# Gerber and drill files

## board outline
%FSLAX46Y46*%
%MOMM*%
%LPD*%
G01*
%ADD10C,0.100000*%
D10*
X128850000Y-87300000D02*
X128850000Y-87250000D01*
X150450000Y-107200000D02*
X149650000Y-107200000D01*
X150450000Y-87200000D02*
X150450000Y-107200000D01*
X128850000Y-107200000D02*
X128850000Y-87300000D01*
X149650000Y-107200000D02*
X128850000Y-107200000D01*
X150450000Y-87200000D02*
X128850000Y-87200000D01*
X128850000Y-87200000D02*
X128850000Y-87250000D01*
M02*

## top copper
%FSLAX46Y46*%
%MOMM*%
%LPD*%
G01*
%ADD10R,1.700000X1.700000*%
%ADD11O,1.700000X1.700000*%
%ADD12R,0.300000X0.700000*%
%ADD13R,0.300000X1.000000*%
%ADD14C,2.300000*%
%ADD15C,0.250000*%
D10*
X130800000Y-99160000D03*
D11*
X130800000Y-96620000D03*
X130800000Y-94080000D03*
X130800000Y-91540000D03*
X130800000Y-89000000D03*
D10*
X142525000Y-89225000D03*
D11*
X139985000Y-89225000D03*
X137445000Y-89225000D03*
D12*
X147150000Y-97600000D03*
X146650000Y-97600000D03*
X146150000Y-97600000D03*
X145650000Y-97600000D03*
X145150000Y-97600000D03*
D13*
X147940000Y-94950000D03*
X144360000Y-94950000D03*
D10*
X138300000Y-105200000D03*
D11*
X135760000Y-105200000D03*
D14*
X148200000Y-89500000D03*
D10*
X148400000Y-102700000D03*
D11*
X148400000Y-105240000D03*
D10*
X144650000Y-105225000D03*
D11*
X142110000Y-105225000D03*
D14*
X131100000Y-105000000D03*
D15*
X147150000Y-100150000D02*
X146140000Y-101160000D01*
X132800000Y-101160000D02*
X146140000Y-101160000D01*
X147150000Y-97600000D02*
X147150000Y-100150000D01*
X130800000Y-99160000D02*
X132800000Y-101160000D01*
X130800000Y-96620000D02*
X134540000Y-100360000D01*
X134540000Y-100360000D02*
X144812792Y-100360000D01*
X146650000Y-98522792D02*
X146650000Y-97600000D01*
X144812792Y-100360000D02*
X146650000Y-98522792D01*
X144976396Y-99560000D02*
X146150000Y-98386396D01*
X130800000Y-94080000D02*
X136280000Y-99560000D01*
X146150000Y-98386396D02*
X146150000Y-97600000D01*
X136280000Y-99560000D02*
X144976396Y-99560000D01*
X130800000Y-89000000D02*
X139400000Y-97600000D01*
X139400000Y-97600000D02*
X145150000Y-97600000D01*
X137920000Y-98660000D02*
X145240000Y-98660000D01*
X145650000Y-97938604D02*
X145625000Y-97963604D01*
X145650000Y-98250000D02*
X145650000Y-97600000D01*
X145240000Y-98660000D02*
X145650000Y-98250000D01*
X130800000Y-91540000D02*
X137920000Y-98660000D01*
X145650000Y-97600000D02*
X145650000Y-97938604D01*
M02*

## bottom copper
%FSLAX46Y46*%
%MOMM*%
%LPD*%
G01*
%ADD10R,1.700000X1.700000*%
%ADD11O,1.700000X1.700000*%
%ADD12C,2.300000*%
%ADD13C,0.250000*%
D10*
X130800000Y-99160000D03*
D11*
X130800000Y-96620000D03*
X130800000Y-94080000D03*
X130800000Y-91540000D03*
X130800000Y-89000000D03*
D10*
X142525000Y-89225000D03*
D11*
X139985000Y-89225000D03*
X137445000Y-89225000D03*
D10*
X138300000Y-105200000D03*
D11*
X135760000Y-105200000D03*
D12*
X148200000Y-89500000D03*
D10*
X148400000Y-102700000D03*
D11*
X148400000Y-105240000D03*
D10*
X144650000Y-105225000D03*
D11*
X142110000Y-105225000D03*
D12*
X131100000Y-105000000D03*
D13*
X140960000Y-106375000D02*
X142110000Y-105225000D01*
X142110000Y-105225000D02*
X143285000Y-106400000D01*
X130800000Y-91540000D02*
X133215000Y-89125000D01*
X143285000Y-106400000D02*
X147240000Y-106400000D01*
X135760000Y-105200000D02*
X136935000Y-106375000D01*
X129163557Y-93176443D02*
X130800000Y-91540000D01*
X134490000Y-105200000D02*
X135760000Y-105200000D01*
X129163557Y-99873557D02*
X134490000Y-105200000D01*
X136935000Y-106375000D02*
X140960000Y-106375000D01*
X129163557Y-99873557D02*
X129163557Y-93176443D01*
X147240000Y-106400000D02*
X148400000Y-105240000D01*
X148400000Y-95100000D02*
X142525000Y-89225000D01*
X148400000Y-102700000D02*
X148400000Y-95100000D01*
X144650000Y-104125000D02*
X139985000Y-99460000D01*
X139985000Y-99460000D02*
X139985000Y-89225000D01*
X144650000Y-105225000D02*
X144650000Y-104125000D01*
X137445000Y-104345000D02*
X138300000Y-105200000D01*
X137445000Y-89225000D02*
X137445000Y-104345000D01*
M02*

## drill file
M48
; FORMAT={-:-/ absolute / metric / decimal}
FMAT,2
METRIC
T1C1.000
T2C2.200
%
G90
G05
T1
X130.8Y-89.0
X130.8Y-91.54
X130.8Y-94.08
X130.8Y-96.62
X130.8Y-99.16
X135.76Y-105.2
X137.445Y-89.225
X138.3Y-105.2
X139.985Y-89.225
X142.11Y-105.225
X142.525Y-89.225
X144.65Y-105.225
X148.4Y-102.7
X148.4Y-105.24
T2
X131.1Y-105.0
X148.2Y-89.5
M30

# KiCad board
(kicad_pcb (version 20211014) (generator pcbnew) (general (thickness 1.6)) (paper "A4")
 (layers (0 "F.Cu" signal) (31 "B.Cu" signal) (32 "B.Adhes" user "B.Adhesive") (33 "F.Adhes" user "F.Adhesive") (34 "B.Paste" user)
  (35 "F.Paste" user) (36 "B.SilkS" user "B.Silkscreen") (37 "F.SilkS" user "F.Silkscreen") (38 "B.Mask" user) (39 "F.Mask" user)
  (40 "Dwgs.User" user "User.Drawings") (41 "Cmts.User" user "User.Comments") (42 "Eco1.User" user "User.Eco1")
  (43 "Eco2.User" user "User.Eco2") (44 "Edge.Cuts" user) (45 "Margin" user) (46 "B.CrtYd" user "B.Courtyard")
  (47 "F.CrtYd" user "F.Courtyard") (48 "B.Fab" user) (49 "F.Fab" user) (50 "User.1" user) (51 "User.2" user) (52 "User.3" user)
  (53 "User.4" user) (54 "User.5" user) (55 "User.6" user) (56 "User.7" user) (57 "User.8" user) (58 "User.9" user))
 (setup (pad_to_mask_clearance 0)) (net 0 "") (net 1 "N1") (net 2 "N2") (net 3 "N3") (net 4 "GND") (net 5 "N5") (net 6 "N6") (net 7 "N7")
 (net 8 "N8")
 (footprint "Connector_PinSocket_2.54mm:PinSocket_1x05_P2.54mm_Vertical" (layer "F.Cu") (at 130.8 99.16 180)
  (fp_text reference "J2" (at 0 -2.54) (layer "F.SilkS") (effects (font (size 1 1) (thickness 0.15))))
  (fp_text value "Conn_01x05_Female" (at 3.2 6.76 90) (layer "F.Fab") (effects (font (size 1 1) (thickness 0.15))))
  (pad "1" thru_hole rect (at 0 0 180) (size 1.7 1.7) (drill 1) (layers *.Cu *.Mask) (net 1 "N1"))
  (pad "2" thru_hole oval (at 0 2.54 180) (size 1.7 1.7) (drill 1) (layers *.Cu *.Mask) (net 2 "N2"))
  (pad "3" thru_hole oval (at 0 5.08 180) (size 1.7 1.7) (drill 1) (layers *.Cu *.Mask) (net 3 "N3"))
  (pad "4" thru_hole oval (at 0 7.62 180) (size 1.7 1.7) (drill 1) (layers *.Cu *.Mask) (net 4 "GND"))
  (pad "5" thru_hole oval (at 0 10.16 180) (size 1.7 1.7) (drill 1) (layers *.Cu *.Mask) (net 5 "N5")))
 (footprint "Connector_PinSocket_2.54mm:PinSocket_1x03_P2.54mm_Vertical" (layer "F.Cu") (at 142.525 89.225 -90)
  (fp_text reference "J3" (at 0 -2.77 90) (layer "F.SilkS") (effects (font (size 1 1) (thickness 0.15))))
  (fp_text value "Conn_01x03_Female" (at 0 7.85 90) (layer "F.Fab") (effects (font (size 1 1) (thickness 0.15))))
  (pad "1" thru_hole rect (at 0 0 270) (size 1.7 1.7) (drill 1) (layers *.Cu *.Mask) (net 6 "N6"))
  (pad "2" thru_hole oval (at 0 2.54 270) (size 1.7 1.7) (drill 1) (layers *.Cu *.Mask) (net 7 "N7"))
  (pad "3" thru_hole oval (at 0 5.08 270) (size 1.7 1.7) (drill 1) (layers *.Cu *.Mask) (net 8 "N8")))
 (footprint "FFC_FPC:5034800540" (layer "F.Cu") (at 146.15 96.1 180)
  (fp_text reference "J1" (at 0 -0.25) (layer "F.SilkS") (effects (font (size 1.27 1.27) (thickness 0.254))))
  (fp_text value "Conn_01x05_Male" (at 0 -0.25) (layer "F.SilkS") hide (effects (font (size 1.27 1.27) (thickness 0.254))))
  (pad "1" smd rect (at -1 -1.5 180) (size 0.3 0.7) (layers "F.Cu" "F.Paste" "F.Mask") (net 1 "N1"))
  (pad "2" smd rect (at -0.5 -1.5 180) (size 0.3 0.7) (layers "F.Cu" "F.Paste" "F.Mask") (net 2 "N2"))
  (pad "3" smd rect (at 0 -1.5 180) (size 0.3 0.7) (layers "F.Cu" "F.Paste" "F.Mask") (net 3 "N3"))
  (pad "4" smd rect (at 0.5 -1.5 180) (size 0.3 0.7) (layers "F.Cu" "F.Paste" "F.Mask") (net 4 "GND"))
  (pad "5" smd rect (at 1 -1.5 180) (size 0.3 0.7) (layers "F.Cu" "F.Paste" "F.Mask") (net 5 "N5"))
  (pad "MP1" smd rect (at -1.79 1.15 180) (size 0.3 1) (layers "F.Cu" "F.Paste" "F.Mask"))
  (pad "MP2" smd rect (at 1.79 1.15 180) (size 0.3 1) (layers "F.Cu" "F.Paste" "F.Mask")))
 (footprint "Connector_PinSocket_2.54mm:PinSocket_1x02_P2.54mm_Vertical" (layer "F.Cu") (at 138.3 105.2 -90)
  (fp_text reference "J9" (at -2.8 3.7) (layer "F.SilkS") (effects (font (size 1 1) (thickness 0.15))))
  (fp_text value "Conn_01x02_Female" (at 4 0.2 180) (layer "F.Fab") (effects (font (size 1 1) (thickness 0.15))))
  (pad "1" thru_hole rect (at 0 0 270) (size 1.7 1.7) (drill 1) (layers *.Cu *.Mask) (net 8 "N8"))
  (pad "2" thru_hole oval (at 0 2.54 270) (size 1.7 1.7) (drill 1) (layers *.Cu *.Mask) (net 4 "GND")))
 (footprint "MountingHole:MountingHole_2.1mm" (layer "F.Cu") (at 148.2 89.5)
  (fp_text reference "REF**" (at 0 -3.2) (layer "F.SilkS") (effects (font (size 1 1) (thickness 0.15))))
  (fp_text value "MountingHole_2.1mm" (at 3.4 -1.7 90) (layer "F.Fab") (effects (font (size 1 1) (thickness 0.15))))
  (pad "" np_thru_hole circle (at 0 0) (size 2.3 2.3) (drill 2.2) (layers F&B.Cu *.Mask)))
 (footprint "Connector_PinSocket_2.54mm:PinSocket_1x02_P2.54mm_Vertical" (layer "F.Cu") (at 148.4 102.7)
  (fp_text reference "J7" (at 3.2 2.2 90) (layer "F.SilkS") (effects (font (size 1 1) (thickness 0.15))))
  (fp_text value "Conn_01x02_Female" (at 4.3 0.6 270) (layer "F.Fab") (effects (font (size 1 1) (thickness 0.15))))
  (pad "1" thru_hole rect (at 0 0) (size 1.7 1.7) (drill 1) (layers *.Cu *.Mask) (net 6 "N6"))
  (pad "2" thru_hole oval (at 0 2.54) (size 1.7 1.7) (drill 1) (layers *.Cu *.Mask) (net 4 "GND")))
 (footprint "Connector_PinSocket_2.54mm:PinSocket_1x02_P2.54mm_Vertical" (layer "F.Cu") (at 144.65 105.225 -90)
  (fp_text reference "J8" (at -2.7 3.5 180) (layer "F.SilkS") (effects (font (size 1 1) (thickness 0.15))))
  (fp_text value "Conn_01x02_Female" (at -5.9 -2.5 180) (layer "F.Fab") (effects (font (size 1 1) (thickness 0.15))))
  (pad "1" thru_hole rect (at 0 0 270) (size 1.7 1.7) (drill 1) (layers *.Cu *.Mask) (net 7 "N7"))
  (pad "2" thru_hole oval (at 0 2.54 270) (size 1.7 1.7) (drill 1) (layers *.Cu *.Mask) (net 4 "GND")))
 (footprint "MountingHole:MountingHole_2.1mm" (layer "F.Cu") (at 131.1 105 180)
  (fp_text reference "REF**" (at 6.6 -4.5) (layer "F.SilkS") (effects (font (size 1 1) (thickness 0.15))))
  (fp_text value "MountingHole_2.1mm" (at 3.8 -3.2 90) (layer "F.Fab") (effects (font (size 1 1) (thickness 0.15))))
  (pad "" np_thru_hole circle (at 0 0 180) (size 2.3 2.3) (drill 2.2) (layers F&B.Cu *.Mask)))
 (gr_line (start 128.85 87.3) (end 128.85 87.25) (layer "Edge.Cuts") (width 0.1))
 (gr_line (start 150.45 107.2) (end 149.65 107.2) (layer "Edge.Cuts") (width 0.1))
 (gr_line (start 150.45 87.2) (end 150.45 107.2) (layer "Edge.Cuts") (width 0.1))
 (gr_line (start 128.85 107.2) (end 128.85 87.3) (layer "Edge.Cuts") (width 0.1))
 (gr_line (start 149.65 107.2) (end 128.85 107.2) (layer "Edge.Cuts") (width 0.1))
 (gr_line (start 150.45 87.2) (end 128.85 87.2) (layer "Edge.Cuts") (width 0.1))
 (gr_line (start 128.85 87.2) (end 128.85 87.25) (layer "Edge.Cuts") (width 0.1))
 (segment (start 147.15 100.15) (end 146.14 101.16) (width 0.25) (layer "F.Cu") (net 1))
 (segment (start 132.8 101.16) (end 146.14 101.16) (width 0.25) (layer "F.Cu") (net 1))
 (segment (start 147.15 97.6) (end 147.15 100.15) (width 0.25) (layer "F.Cu") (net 1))
 (segment (start 130.8 99.16) (end 132.8 101.16) (width 0.25) (layer "F.Cu") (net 1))
 (segment (start 130.8 96.62) (end 134.54 100.36) (width 0.25) (layer "F.Cu") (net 2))
 (segment (start 134.54 100.36) (end 144.812792 100.36) (width 0.25) (layer "F.Cu") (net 2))
 (segment (start 146.65 98.522792) (end 146.65 97.6) (width 0.25) (layer "F.Cu") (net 2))
 (segment (start 144.812792 100.36) (end 146.65 98.522792) (width 0.25) (layer "F.Cu") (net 2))
 (segment (start 144.976396 99.56) (end 146.15 98.386396) (width 0.25) (layer "F.Cu") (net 3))
 (segment (start 130.8 94.08) (end 136.28 99.56) (width 0.25) (layer "F.Cu") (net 3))
 (segment (start 146.15 98.386396) (end 146.15 97.6) (width 0.25) (layer "F.Cu") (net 3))
 (segment (start 136.28 99.56) (end 144.976396 99.56) (width 0.25) (layer "F.Cu") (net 3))
 (segment (start 130.8 89) (end 139.4 97.6) (width 0.25) (layer "F.Cu") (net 5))
 (segment (start 139.4 97.6) (end 145.15 97.6) (width 0.25) (layer "F.Cu") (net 5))
 (segment (start 137.92 98.66) (end 145.24 98.66) (width 0.25) (layer "F.Cu") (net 4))
 (segment (start 145.65 97.938604) (end 145.625 97.963604) (width 0.25) (layer "F.Cu") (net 4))
 (segment (start 145.65 98.25) (end 145.65 97.6) (width 0.25) (layer "F.Cu") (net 4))
 (segment (start 145.24 98.66) (end 145.65 98.25) (width 0.25) (layer "F.Cu") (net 4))
 (segment (start 130.8 91.54) (end 137.92 98.66) (width 0.25) (layer "F.Cu") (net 4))
 (segment (start 145.65 97.6) (end 145.65 97.938604) (width 0.25) (layer "F.Cu") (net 4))
 (segment (start 140.96 106.375) (end 142.11 105.225) (width 0.25) (layer "B.Cu") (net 4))
 (segment (start 142.11 105.225) (end 143.285 106.4) (width 0.25) (layer "B.Cu") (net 4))
 (segment (start 130.8 91.54) (end 133.215 89.125) (width 0.25) (layer "B.Cu") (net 4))
 (segment (start 143.285 106.4) (end 147.24 106.4) (width 0.25) (layer "B.Cu") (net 4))
 (segment (start 135.76 105.2) (end 136.935 106.375) (width 0.25) (layer "B.Cu") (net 4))
 (segment (start 129.163557 93.176443) (end 130.8 91.54) (width 0.25) (layer "B.Cu") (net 4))
 (segment (start 134.49 105.2) (end 135.76 105.2) (width 0.25) (layer "B.Cu") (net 4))
 (segment (start 129.163557 99.873557) (end 134.49 105.2) (width 0.25) (layer "B.Cu") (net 4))
 (segment (start 136.935 106.375) (end 140.96 106.375) (width 0.25) (layer "B.Cu") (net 4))
 (segment (start 129.163557 99.873557) (end 129.163557 93.176443) (width 0.25) (layer "B.Cu") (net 4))
 (segment (start 147.24 106.4) (end 148.4 105.24) (width 0.25) (layer "B.Cu") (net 4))
 (segment (start 148.4 95.1) (end 142.525 89.225) (width 0.25) (layer "B.Cu") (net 6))
 (segment (start 148.4 102.7) (end 148.4 95.1) (width 0.25) (layer "B.Cu") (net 6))
 (segment (start 144.65 104.125) (end 139.985 99.46) (width 0.25) (layer "B.Cu") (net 7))
 (segment (start 139.985 99.46) (end 139.985 89.225) (width 0.25) (layer "B.Cu") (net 7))
 (segment (start 144.65 105.225) (end 144.65 104.125) (width 0.25) (layer "B.Cu") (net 7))
 (segment (start 137.445 104.345) (end 138.3 105.2) (width 0.25) (layer "B.Cu") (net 8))
 (segment (start 137.445 89.225) (end 137.445 104.345) (width 0.25) (layer "B.Cu") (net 8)))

